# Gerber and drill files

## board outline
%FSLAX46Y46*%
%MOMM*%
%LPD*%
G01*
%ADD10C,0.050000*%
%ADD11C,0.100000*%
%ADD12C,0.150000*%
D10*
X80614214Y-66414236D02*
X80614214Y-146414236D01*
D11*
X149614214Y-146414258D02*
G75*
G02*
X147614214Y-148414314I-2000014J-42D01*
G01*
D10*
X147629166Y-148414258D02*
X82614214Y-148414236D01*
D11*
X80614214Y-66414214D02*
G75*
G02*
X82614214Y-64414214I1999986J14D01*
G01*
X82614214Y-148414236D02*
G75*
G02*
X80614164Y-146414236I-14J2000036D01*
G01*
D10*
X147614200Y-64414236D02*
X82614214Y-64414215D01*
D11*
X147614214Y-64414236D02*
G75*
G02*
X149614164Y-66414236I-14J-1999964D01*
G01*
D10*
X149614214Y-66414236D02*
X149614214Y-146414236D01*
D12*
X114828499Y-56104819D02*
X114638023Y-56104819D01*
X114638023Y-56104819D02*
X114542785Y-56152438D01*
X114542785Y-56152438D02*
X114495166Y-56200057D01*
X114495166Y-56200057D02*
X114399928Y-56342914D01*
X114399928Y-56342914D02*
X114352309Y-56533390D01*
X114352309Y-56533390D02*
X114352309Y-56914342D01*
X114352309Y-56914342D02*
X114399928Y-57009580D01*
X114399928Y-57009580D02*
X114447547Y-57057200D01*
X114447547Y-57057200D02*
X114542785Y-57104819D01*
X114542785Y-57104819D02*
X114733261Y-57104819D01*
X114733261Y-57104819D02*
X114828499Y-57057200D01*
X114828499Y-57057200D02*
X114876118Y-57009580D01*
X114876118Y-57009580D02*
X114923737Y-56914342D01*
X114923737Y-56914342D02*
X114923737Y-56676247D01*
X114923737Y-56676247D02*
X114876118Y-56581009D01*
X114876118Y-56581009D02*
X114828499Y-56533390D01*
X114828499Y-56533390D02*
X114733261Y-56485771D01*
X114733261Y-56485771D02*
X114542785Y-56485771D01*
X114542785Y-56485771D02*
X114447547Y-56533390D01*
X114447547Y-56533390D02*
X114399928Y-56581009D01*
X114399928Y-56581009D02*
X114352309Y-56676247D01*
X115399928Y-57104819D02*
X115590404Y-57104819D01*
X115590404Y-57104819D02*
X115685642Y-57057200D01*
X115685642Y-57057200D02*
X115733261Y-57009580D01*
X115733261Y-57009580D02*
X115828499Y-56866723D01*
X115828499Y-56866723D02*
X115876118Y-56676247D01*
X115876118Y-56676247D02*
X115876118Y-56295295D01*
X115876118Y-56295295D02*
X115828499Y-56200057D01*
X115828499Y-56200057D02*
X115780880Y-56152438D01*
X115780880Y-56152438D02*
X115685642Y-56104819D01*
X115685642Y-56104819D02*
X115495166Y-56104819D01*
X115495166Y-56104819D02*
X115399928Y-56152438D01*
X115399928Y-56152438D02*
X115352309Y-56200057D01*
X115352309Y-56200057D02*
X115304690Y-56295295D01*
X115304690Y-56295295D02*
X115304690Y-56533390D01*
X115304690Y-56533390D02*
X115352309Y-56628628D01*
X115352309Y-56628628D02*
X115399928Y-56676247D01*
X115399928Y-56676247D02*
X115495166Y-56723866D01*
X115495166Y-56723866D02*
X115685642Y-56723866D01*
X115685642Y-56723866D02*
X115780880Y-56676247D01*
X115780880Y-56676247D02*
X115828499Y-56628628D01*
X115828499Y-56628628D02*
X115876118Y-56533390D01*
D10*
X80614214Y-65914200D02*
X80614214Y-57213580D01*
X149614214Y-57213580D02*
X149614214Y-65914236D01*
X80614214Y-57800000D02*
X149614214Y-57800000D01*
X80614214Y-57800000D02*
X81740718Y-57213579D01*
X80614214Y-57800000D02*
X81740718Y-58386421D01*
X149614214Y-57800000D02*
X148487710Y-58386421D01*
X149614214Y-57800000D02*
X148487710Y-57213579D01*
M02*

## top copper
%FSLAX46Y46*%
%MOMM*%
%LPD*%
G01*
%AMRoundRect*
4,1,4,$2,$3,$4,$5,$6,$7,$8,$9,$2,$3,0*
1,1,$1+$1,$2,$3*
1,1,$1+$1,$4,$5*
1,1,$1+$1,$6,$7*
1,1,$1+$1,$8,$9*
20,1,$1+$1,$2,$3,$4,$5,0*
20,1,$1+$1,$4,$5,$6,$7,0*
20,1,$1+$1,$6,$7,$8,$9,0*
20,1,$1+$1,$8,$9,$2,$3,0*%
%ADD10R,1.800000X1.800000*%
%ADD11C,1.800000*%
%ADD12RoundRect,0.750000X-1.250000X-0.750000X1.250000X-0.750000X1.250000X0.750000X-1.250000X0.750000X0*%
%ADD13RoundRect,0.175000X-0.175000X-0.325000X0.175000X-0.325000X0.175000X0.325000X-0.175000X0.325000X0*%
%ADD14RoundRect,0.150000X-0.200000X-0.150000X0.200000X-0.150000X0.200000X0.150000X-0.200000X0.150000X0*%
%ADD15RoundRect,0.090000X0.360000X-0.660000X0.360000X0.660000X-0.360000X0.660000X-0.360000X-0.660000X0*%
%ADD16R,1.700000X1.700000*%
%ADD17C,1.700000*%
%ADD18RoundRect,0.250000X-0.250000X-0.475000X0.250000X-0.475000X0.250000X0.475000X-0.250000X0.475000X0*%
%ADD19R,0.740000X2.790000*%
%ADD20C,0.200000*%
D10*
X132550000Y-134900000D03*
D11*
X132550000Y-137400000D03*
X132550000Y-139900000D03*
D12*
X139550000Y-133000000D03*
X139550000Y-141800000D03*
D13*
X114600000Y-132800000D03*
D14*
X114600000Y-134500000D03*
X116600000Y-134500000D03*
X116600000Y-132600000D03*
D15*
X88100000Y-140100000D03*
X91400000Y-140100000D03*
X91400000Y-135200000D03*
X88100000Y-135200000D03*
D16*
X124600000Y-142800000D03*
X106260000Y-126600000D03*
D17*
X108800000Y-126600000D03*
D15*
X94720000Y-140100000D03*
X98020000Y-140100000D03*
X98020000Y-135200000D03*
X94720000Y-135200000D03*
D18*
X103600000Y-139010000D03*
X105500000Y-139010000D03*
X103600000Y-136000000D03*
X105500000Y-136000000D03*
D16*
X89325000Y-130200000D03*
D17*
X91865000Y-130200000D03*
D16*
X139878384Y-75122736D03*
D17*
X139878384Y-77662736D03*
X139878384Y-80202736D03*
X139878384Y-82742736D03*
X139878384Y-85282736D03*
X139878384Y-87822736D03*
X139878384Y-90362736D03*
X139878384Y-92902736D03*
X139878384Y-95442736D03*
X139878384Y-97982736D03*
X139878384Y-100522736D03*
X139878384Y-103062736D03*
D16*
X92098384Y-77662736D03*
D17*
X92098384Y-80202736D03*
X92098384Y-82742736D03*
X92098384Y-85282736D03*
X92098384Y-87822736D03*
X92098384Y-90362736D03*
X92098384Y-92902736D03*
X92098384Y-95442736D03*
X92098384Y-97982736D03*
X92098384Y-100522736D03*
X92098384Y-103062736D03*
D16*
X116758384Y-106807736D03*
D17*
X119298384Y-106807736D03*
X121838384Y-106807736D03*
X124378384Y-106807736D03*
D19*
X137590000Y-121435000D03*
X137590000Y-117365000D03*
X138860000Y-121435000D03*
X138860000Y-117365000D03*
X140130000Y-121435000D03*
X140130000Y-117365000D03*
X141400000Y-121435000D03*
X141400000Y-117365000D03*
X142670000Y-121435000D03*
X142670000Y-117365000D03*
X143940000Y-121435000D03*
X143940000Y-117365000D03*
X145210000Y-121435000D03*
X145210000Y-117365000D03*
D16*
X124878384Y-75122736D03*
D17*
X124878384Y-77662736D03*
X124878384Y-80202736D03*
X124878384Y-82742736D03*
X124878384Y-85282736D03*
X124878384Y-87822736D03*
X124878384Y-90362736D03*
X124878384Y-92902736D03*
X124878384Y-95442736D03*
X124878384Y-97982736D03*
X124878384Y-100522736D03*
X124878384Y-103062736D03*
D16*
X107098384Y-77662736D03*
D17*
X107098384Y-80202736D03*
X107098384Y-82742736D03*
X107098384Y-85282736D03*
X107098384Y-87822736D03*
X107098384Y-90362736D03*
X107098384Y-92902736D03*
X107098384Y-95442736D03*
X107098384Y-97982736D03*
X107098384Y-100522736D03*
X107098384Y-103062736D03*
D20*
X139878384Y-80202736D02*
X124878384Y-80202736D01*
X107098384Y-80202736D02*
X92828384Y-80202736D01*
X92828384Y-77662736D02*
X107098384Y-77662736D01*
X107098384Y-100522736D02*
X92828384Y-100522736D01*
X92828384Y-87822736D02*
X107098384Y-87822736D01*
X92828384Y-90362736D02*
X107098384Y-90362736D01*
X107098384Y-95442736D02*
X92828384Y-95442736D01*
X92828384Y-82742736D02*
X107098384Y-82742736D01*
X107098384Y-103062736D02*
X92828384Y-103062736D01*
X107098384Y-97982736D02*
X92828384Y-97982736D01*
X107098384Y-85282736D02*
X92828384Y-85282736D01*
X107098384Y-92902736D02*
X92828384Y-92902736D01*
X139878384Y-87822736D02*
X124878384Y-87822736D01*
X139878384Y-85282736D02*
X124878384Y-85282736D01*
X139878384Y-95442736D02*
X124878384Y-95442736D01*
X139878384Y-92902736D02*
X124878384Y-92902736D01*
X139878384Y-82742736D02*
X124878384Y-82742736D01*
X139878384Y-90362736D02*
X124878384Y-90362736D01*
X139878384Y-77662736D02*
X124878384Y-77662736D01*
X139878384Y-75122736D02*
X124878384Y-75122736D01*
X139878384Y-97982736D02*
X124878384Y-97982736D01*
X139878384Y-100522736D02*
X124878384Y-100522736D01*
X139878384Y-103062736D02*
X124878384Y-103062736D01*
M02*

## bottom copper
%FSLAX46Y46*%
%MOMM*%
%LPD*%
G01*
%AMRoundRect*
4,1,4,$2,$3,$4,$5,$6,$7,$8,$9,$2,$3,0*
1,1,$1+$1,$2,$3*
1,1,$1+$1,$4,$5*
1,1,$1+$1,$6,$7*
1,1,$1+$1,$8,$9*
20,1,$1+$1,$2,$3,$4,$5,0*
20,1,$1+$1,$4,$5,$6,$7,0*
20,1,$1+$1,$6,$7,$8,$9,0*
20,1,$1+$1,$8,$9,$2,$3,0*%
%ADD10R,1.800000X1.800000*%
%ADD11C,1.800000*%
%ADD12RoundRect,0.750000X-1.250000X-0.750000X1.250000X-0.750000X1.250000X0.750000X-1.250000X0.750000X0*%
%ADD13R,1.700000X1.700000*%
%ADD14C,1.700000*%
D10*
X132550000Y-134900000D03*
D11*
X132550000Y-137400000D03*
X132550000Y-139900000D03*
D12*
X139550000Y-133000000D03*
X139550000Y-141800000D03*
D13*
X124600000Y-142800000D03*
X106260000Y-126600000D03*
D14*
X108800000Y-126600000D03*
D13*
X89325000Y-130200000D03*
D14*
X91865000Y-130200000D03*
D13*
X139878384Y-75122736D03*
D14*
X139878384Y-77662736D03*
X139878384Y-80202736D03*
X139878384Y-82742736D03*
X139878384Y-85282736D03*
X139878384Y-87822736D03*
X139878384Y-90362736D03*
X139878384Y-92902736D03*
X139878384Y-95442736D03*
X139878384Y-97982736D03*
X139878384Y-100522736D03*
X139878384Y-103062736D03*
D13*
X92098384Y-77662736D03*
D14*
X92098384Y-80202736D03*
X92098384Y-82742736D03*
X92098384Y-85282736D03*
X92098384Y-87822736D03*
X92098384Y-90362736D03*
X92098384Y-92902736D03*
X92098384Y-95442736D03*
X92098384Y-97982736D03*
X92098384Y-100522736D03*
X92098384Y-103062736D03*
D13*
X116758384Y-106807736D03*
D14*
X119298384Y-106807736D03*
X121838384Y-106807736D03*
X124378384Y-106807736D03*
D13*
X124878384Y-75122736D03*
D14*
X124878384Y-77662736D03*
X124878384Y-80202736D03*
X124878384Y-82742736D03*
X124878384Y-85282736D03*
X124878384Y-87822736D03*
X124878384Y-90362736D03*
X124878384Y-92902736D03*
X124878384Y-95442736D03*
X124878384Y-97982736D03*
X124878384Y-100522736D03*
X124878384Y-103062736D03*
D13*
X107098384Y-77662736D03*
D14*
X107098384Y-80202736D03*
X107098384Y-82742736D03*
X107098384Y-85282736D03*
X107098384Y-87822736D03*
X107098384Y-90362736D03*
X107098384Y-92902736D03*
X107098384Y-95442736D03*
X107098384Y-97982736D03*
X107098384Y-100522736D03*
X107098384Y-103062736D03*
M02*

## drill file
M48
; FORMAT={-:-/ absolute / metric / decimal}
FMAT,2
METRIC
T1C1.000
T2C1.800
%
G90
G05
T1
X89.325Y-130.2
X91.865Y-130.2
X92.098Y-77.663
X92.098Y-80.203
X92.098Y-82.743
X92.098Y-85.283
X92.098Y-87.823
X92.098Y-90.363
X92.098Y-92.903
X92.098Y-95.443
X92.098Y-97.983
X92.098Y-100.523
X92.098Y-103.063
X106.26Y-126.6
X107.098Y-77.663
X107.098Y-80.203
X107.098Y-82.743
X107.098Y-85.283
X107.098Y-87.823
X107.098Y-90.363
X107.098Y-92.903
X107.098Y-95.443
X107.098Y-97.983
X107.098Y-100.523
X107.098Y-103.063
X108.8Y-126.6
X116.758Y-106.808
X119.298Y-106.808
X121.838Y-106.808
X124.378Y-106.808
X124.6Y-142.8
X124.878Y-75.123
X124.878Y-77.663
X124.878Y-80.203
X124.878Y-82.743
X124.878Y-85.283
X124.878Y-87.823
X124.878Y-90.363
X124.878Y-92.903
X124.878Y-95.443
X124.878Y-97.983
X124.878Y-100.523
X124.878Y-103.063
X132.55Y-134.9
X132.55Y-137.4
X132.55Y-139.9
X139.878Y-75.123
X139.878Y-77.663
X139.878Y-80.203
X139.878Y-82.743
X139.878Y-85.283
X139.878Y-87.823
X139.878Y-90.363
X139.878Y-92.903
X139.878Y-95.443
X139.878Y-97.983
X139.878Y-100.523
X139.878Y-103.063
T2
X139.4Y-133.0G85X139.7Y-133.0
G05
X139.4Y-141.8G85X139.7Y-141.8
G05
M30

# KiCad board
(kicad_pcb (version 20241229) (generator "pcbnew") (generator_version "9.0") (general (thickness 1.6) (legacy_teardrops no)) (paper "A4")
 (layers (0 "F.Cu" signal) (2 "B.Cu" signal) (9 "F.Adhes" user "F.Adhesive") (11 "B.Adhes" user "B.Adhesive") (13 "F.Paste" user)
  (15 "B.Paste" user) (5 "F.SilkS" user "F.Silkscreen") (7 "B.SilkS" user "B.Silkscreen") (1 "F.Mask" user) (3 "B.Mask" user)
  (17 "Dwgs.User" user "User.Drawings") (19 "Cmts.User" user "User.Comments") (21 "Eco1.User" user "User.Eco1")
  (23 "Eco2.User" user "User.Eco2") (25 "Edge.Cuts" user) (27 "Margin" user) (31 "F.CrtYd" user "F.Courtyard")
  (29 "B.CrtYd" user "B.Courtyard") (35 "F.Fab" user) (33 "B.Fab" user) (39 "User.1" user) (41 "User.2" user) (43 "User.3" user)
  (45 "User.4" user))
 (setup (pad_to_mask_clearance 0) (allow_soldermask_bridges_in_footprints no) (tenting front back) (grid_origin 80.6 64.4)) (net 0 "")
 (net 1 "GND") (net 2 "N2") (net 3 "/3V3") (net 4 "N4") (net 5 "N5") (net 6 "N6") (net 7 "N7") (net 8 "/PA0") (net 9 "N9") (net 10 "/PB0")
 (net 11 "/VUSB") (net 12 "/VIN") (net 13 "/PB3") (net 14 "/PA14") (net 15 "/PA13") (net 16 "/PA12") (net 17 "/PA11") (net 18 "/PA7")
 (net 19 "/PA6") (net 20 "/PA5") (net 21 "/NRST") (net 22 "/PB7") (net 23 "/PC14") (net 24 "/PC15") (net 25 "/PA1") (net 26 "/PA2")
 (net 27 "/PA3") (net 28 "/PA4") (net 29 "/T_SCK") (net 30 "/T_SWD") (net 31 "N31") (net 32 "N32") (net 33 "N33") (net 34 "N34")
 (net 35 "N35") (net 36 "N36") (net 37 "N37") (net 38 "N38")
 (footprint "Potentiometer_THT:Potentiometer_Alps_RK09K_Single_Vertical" (layer "F.Cu") (at 132.55 134.9)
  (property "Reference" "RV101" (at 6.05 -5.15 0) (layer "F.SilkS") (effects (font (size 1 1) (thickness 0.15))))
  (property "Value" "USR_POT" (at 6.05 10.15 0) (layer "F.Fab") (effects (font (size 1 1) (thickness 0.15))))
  (pad "1" thru_hole rect (at 0 0) (size 1.8 1.8) (drill 1) (layers "*.Cu" "*.Mask") (remove_unused_layers no) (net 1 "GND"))
  (pad "2" thru_hole circle (at 0 2.5) (size 1.8 1.8) (drill 1) (layers "*.Cu" "*.Mask") (remove_unused_layers no) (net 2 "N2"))
  (pad "3" thru_hole circle (at 0 5) (size 1.8 1.8) (drill 1) (layers "*.Cu" "*.Mask") (remove_unused_layers no) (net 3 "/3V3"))
  (pad "MP" thru_hole roundrect (at 7 -1.9) (size 4 3) (drill oval 2.1 1.8) (layers "*.Cu" "*.Mask") (remove_unused_layers no)
   (roundrect_rratio 0.25))
  (pad "MP" thru_hole roundrect (at 7 6.9) (size 4 3) (drill oval 2.1 1.8) (layers "*.Cu" "*.Mask") (remove_unused_layers no)
   (roundrect_rratio 0.25)))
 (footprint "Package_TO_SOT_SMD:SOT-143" (layer "F.Cu") (at 115.6 133.55)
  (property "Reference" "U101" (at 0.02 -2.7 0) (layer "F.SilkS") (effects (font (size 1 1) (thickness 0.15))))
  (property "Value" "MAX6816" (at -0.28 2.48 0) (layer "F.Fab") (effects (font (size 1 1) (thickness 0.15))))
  (pad "1" smd roundrect (at -1 -0.75) (size 0.7 1) (layers "F.Cu" "F.Mask" "F.Paste") (roundrect_rratio 0.25) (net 1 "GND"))
  (pad "2" smd roundrect (at -1 0.95) (size 0.7 0.6) (layers "F.Cu" "F.Mask" "F.Paste") (roundrect_rratio 0.25) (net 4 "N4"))
  (pad "3" smd roundrect (at 1 0.95) (size 0.7 0.6) (layers "F.Cu" "F.Mask" "F.Paste") (roundrect_rratio 0.25) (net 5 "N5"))
  (pad "4" smd roundrect (at 1 -0.95) (size 0.7 0.6) (layers "F.Cu" "F.Mask" "F.Paste") (roundrect_rratio 0.25) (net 3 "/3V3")))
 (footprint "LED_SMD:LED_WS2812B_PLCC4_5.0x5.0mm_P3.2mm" (layer "F.Cu") (at 89.75 137.65 90)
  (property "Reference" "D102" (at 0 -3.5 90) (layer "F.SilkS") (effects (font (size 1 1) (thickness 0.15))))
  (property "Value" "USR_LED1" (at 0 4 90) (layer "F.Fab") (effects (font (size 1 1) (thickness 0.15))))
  (pad "1" smd roundrect (at -2.45 -1.65 90) (size 1.5 0.9) (layers "F.Cu" "F.Mask" "F.Paste") (roundrect_rratio 0.1) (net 3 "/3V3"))
  (pad "2" smd roundrect (at -2.45 1.65 90) (size 1.5 0.9) (layers "F.Cu" "F.Mask" "F.Paste") (roundrect_rratio 0.1) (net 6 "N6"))
  (pad "3" smd roundrect (at 2.45 1.65 90) (size 1.5 0.9) (layers "F.Cu" "F.Mask" "F.Paste") (roundrect_rratio 0.1) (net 1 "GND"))
  (pad "4" smd roundrect (at 2.45 -1.65 90) (size 1.5 0.9) (layers "F.Cu" "F.Mask" "F.Paste") (roundrect_rratio 0.1) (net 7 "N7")))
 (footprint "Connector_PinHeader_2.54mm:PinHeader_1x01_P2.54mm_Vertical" (layer "F.Cu") (at 124.6 142.8)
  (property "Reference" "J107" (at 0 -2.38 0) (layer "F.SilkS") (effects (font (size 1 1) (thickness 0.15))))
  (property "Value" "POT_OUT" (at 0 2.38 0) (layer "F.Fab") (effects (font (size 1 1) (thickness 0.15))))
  (pad "1" thru_hole rect (at 0 0) (size 1.7 1.7) (drill 1) (layers "*.Cu" "*.Mask") (remove_unused_layers no) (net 2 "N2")))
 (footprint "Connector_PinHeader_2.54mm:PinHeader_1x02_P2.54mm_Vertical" (layer "F.Cu") (at 106.26 126.6 90)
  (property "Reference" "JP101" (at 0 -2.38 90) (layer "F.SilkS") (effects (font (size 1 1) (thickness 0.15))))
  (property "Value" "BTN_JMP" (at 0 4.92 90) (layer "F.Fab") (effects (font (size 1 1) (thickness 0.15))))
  (pad "1" thru_hole rect (at 0 0 90) (size 1.7 1.7) (drill 1) (layers "*.Cu" "*.Mask") (remove_unused_layers no) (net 5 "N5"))
  (pad "2" thru_hole circle (at 0 2.54 90) (size 1.7 1.7) (drill 1) (layers "*.Cu" "*.Mask") (remove_unused_layers no) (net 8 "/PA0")))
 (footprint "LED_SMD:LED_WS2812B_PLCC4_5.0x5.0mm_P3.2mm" (layer "F.Cu") (at 96.37 137.65 90)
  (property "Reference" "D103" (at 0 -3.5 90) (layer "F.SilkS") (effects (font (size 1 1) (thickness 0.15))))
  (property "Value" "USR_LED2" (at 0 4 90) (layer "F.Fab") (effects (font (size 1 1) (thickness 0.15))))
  (pad "1" smd roundrect (at -2.45 -1.65 90) (size 1.5 0.9) (layers "F.Cu" "F.Mask" "F.Paste") (roundrect_rratio 0.1) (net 3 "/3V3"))
  (pad "2" smd roundrect (at -2.45 1.65 90) (size 1.5 0.9) (layers "F.Cu" "F.Mask" "F.Paste") (roundrect_rratio 0.1) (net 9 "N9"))
  (pad "3" smd roundrect (at 2.45 1.65 90) (size 1.5 0.9) (layers "F.Cu" "F.Mask" "F.Paste") (roundrect_rratio 0.1) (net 1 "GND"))
  (pad "4" smd roundrect (at 2.45 -1.65 90) (size 1.5 0.9) (layers "F.Cu" "F.Mask" "F.Paste") (roundrect_rratio 0.1) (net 6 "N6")))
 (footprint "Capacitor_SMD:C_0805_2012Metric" (layer "F.Cu") (at 104.55 139.01)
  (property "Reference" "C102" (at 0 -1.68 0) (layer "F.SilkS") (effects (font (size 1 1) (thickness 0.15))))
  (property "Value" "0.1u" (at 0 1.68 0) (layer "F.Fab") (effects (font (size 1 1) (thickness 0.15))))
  (pad "1" smd roundrect (at -0.95 0) (size 1 1.45) (layers "F.Cu" "F.Mask" "F.Paste") (roundrect_rratio 0.25) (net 3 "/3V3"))
  (pad "2" smd roundrect (at 0.95 0) (size 1 1.45) (layers "F.Cu" "F.Mask" "F.Paste") (roundrect_rratio 0.25) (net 1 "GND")))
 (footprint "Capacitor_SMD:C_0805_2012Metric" (layer "F.Cu") (at 104.55 136)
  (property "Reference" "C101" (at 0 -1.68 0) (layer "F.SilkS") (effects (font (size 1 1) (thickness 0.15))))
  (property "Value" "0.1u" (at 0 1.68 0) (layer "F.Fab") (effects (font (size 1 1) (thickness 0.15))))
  (pad "1" smd roundrect (at -0.95 0) (size 1 1.45) (layers "F.Cu" "F.Mask" "F.Paste") (roundrect_rratio 0.25) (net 3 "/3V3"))
  (pad "2" smd roundrect (at 0.95 0) (size 1 1.45) (layers "F.Cu" "F.Mask" "F.Paste") (roundrect_rratio 0.25) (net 1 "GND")))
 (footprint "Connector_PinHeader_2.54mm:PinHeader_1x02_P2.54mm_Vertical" (layer "F.Cu") (at 89.325 130.2 90)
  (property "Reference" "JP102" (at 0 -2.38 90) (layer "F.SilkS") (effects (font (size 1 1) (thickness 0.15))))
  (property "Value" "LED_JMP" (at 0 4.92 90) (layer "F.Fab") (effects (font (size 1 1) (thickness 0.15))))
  (pad "1" thru_hole rect (at 0 0 90) (size 1.7 1.7) (drill 1) (layers "*.Cu" "*.Mask") (remove_unused_layers no) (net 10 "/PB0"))
  (pad "2" thru_hole circle (at 0 2.54 90) (size 1.7 1.7) (drill 1) (layers "*.Cu" "*.Mask") (remove_unused_layers no) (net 7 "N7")))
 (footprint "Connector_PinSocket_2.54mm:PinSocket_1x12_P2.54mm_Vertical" (layer "F.Cu") (at 139.878384 75.122736)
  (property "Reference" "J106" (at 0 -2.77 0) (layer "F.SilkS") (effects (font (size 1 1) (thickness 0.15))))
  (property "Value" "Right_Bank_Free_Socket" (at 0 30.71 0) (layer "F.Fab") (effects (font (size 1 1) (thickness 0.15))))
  (pad "1" thru_hole rect (at 0 0) (size 1.7 1.7) (drill 1) (layers "*.Cu" "*.Mask") (remove_unused_layers no) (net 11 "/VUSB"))
  (pad "2" thru_hole circle (at 0 2.54) (size 1.7 1.7) (drill 1) (layers "*.Cu" "*.Mask") (remove_unused_layers no) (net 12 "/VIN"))
  (pad "3" thru_hole circle (at 0 5.08) (size 1.7 1.7) (drill 1) (layers "*.Cu" "*.Mask") (remove_unused_layers no) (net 1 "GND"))
  (pad "4" thru_hole circle (at 0 7.62) (size 1.7 1.7) (drill 1) (layers "*.Cu" "*.Mask") (remove_unused_layers no) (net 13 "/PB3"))
  (pad "5" thru_hole circle (at 0 10.16) (size 1.7 1.7) (drill 1) (layers "*.Cu" "*.Mask") (remove_unused_layers no) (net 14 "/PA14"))
  (pad "6" thru_hole circle (at 0 12.7) (size 1.7 1.7) (drill 1) (layers "*.Cu" "*.Mask") (remove_unused_layers no) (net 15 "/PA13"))
  (pad "7" thru_hole circle (at 0 15.24) (size 1.7 1.7) (drill 1) (layers "*.Cu" "*.Mask") (remove_unused_layers no) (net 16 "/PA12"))
  (pad "8" thru_hole circle (at 0 17.78) (size 1.7 1.7) (drill 1) (layers "*.Cu" "*.Mask") (remove_unused_layers no) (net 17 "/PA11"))
  (pad "9" thru_hole circle (at 0 20.32) (size 1.7 1.7) (drill 1) (layers "*.Cu" "*.Mask") (remove_unused_layers no) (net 10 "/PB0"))
  (pad "10" thru_hole circle (at 0 22.86) (size 1.7 1.7) (drill 1) (layers "*.Cu" "*.Mask") (remove_unused_layers no) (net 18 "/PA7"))
  (pad "11" thru_hole circle (at 0 25.4) (size 1.7 1.7) (drill 1) (layers "*.Cu" "*.Mask") (remove_unused_layers no) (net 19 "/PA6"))
  (pad "12" thru_hole circle (at 0 27.94) (size 1.7 1.7) (drill 1) (layers "*.Cu" "*.Mask") (remove_unused_layers no) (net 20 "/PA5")))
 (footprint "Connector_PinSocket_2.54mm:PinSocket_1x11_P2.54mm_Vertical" (layer "F.Cu") (at 92.098384 77.662736)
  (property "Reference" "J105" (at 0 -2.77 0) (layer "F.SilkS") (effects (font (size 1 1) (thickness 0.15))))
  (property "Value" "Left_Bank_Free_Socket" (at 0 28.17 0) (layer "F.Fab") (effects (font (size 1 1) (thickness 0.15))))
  (pad "1" thru_hole rect (at 0 0) (size 1.7 1.7) (drill 1) (layers "*.Cu" "*.Mask") (remove_unused_layers no) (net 3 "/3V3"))
  (pad "2" thru_hole circle (at 0 2.54) (size 1.7 1.7) (drill 1) (layers "*.Cu" "*.Mask") (remove_unused_layers no) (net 1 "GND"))
  (pad "3" thru_hole circle (at 0 5.08) (size 1.7 1.7) (drill 1) (layers "*.Cu" "*.Mask") (remove_unused_layers no) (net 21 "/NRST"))
  (pad "4" thru_hole circle (at 0 7.62) (size 1.7 1.7) (drill 1) (layers "*.Cu" "*.Mask") (remove_unused_layers no) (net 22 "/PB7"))
  (pad "5" thru_hole circle (at 0 10.16) (size 1.7 1.7) (drill 1) (layers "*.Cu" "*.Mask") (remove_unused_layers no) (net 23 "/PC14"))
  (pad "6" thru_hole circle (at 0 12.7) (size 1.7 1.7) (drill 1) (layers "*.Cu" "*.Mask") (remove_unused_layers no) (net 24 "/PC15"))
  (pad "7" thru_hole circle (at 0 15.24) (size 1.7 1.7) (drill 1) (layers "*.Cu" "*.Mask") (remove_unused_layers no) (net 8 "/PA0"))
  (pad "8" thru_hole circle (at 0 17.78) (size 1.7 1.7) (drill 1) (layers "*.Cu" "*.Mask") (remove_unused_layers no) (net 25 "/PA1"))
  (pad "9" thru_hole circle (at 0 20.32) (size 1.7 1.7) (drill 1) (layers "*.Cu" "*.Mask") (remove_unused_layers no) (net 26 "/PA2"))
  (pad "10" thru_hole circle (at 0 22.86) (size 1.7 1.7) (drill 1) (layers "*.Cu" "*.Mask") (remove_unused_layers no) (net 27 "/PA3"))
  (pad "11" thru_hole circle (at 0 25.4) (size 1.7 1.7) (drill 1) (layers "*.Cu" "*.Mask") (remove_unused_layers no) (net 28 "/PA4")))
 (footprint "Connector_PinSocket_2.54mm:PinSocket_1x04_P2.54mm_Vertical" (layer "F.Cu") (at 116.758384 106.807736 90)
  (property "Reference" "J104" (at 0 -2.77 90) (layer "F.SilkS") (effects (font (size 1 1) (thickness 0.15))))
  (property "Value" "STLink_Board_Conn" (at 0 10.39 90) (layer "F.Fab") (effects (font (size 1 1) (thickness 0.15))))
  (pad "1" thru_hole rect (at 0 0 90) (size 1.7 1.7) (drill 1) (layers "*.Cu" "*.Mask") (remove_unused_layers no) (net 3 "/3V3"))
  (pad "2" thru_hole circle (at 0 2.54 90) (size 1.7 1.7) (drill 1) (layers "*.Cu" "*.Mask") (remove_unused_layers no) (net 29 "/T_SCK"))
  (pad "3" thru_hole circle (at 0 5.08 90) (size 1.7 1.7) (drill 1) (layers "*.Cu" "*.Mask") (remove_unused_layers no) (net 1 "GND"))
  (pad "4" thru_hole circle (at 0 7.62 90) (size 1.7 1.7) (drill 1) (layers "*.Cu" "*.Mask") (remove_unused_layers no) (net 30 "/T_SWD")))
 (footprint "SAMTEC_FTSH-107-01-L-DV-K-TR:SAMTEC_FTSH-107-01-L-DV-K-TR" (layer "F.Cu") (at 141.4 119.4)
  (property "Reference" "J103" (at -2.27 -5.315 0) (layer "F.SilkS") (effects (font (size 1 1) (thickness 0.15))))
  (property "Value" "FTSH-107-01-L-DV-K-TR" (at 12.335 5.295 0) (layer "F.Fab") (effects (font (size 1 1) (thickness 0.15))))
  (pad "1" smd rect (at -3.81 2.035) (size 0.74 2.79) (layers "F.Cu" "F.Mask" "F.Paste") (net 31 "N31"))
  (pad "2" smd rect (at -3.81 -2.035) (size 0.74 2.79) (layers "F.Cu" "F.Mask" "F.Paste") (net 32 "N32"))
  (pad "3" smd rect (at -2.54 2.035) (size 0.74 2.79) (layers "F.Cu" "F.Mask" "F.Paste") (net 3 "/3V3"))
  (pad "4" smd rect (at -2.54 -2.035) (size 0.74 2.79) (layers "F.Cu" "F.Mask" "F.Paste") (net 30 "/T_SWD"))
  (pad "5" smd rect (at -1.27 2.035) (size 0.74 2.79) (layers "F.Cu" "F.Mask" "F.Paste") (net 1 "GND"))
  (pad "6" smd rect (at -1.27 -2.035) (size 0.74 2.79) (layers "F.Cu" "F.Mask" "F.Paste") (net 29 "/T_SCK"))
  (pad "7" smd rect (at 0 2.035) (size 0.74 2.79) (layers "F.Cu" "F.Mask" "F.Paste") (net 1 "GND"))
  (pad "8" smd rect (at 0 -2.035) (size 0.74 2.79) (layers "F.Cu" "F.Mask" "F.Paste") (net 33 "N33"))
  (pad "9" smd rect (at 1.27 2.035) (size 0.74 2.79) (layers "F.Cu" "F.Mask" "F.Paste") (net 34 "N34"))
  (pad "10" smd rect (at 1.27 -2.035) (size 0.74 2.79) (layers "F.Cu" "F.Mask" "F.Paste") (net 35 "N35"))
  (pad "11" smd rect (at 2.54 2.035) (size 0.74 2.79) (layers "F.Cu" "F.Mask" "F.Paste") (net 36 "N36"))
  (pad "12" smd rect (at 2.54 -2.035) (size 0.74 2.79) (layers "F.Cu" "F.Mask" "F.Paste") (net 21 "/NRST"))
  (pad "13" smd rect (at 3.81 2.035) (size 0.74 2.79) (layers "F.Cu" "F.Mask" "F.Paste") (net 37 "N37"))
  (pad "14" smd rect (at 3.81 -2.035) (size 0.74 2.79) (layers "F.Cu" "F.Mask" "F.Paste") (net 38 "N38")))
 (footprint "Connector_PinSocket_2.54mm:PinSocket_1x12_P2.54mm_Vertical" (layer "F.Cu") (at 124.878384 75.122736)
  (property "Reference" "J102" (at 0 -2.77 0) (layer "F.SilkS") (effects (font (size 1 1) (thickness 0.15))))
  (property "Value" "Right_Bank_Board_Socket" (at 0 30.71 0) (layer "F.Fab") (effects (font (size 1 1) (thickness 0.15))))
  (pad "1" thru_hole rect (at 0 0) (size 1.7 1.7) (drill 1) (layers "*.Cu" "*.Mask") (remove_unused_layers no) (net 11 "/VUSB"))
  (pad "2" thru_hole circle (at 0 2.54) (size 1.7 1.7) (drill 1) (layers "*.Cu" "*.Mask") (remove_unused_layers no) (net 12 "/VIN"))
  (pad "3" thru_hole circle (at 0 5.08) (size 1.7 1.7) (drill 1) (layers "*.Cu" "*.Mask") (remove_unused_layers no) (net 1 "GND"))
  (pad "4" thru_hole circle (at 0 7.62) (size 1.7 1.7) (drill 1) (layers "*.Cu" "*.Mask") (remove_unused_layers no) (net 13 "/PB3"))
  (pad "5" thru_hole circle (at 0 10.16) (size 1.7 1.7) (drill 1) (layers "*.Cu" "*.Mask") (remove_unused_layers no) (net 14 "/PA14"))
  (pad "6" thru_hole circle (at 0 12.7) (size 1.7 1.7) (drill 1) (layers "*.Cu" "*.Mask") (remove_unused_layers no) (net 15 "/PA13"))
  (pad "7" thru_hole circle (at 0 15.24) (size 1.7 1.7) (drill 1) (layers "*.Cu" "*.Mask") (remove_unused_layers no) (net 16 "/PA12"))
  (pad "8" thru_hole circle (at 0 17.78) (size 1.7 1.7) (drill 1) (layers "*.Cu" "*.Mask") (remove_unused_layers no) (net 17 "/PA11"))
  (pad "9" thru_hole circle (at 0 20.32) (size 1.7 1.7) (drill 1) (layers "*.Cu" "*.Mask") (remove_unused_layers no) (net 10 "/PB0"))
  (pad "10" thru_hole circle (at 0 22.86) (size 1.7 1.7) (drill 1) (layers "*.Cu" "*.Mask") (remove_unused_layers no) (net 18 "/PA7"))
  (pad "11" thru_hole circle (at 0 25.4) (size 1.7 1.7) (drill 1) (layers "*.Cu" "*.Mask") (remove_unused_layers no) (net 19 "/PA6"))
  (pad "12" thru_hole circle (at 0 27.94) (size 1.7 1.7) (drill 1) (layers "*.Cu" "*.Mask") (remove_unused_layers no) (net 20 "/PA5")))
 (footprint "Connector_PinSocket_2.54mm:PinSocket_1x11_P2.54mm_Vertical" (layer "F.Cu") (at 107.098384 77.662736)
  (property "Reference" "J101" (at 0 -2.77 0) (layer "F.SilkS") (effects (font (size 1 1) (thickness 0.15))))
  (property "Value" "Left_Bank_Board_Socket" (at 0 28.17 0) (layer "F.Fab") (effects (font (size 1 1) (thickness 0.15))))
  (pad "1" thru_hole rect (at 0 0) (size 1.7 1.7) (drill 1) (layers "*.Cu" "*.Mask") (remove_unused_layers no) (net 3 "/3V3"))
  (pad "2" thru_hole circle (at 0 2.54) (size 1.7 1.7) (drill 1) (layers "*.Cu" "*.Mask") (remove_unused_layers no) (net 1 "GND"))
  (pad "3" thru_hole circle (at 0 5.08) (size 1.7 1.7) (drill 1) (layers "*.Cu" "*.Mask") (remove_unused_layers no) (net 21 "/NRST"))
  (pad "4" thru_hole circle (at 0 7.62) (size 1.7 1.7) (drill 1) (layers "*.Cu" "*.Mask") (remove_unused_layers no) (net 22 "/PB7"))
  (pad "5" thru_hole circle (at 0 10.16) (size 1.7 1.7) (drill 1) (layers "*.Cu" "*.Mask") (remove_unused_layers no) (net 23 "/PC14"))
  (pad "6" thru_hole circle (at 0 12.7) (size 1.7 1.7) (drill 1) (layers "*.Cu" "*.Mask") (remove_unused_layers no) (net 24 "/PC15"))
  (pad "7" thru_hole circle (at 0 15.24) (size 1.7 1.7) (drill 1) (layers "*.Cu" "*.Mask") (remove_unused_layers no) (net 8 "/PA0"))
  (pad "8" thru_hole circle (at 0 17.78) (size 1.7 1.7) (drill 1) (layers "*.Cu" "*.Mask") (remove_unused_layers no) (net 25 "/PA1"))
  (pad "9" thru_hole circle (at 0 20.32) (size 1.7 1.7) (drill 1) (layers "*.Cu" "*.Mask") (remove_unused_layers no) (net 26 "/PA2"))
  (pad "10" thru_hole circle (at 0 22.86) (size 1.7 1.7) (drill 1) (layers "*.Cu" "*.Mask") (remove_unused_layers no) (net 27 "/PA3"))
  (pad "11" thru_hole circle (at 0 25.4) (size 1.7 1.7) (drill 1) (layers "*.Cu" "*.Mask") (remove_unused_layers no) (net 28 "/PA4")))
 (gr_line (start 80.614214 66.414236) (end 80.614214 146.414236) (stroke (width 0.05) (type solid)) (layer "Edge.Cuts"))
 (gr_arc (start 149.614214 146.414258) (mid 149.028428 147.828472) (end 147.614214 148.414258) (stroke (width 0.1) (type solid))
  (layer "Edge.Cuts"))
 (gr_line (start 147.629166 148.414258) (end 82.614214 148.414236) (stroke (width 0.05) (type default)) (layer "Edge.Cuts"))
 (gr_arc (start 80.614214 66.414214) (mid 81.2 65) (end 82.614214 64.414214) (stroke (width 0.1) (type solid)) (layer "Edge.Cuts"))
 (gr_arc (start 82.614214 148.414236) (mid 81.2 147.82845) (end 80.614214 146.414236) (stroke (width 0.1) (type solid)) (layer "Edge.Cuts"))
 (gr_line (start 147.6142 64.414236) (end 82.614214 64.414215) (stroke (width 0.05) (type default)) (layer "Edge.Cuts"))
 (gr_arc (start 147.614214 64.414236) (mid 149.028428 65.000022) (end 149.614214 66.414236) (stroke (width 0.1) (type solid))
  (layer "Edge.Cuts"))
 (gr_line (start 149.614214 66.414236) (end 149.614214 146.414236) (stroke (width 0.05) (type solid)) (layer "Edge.Cuts"))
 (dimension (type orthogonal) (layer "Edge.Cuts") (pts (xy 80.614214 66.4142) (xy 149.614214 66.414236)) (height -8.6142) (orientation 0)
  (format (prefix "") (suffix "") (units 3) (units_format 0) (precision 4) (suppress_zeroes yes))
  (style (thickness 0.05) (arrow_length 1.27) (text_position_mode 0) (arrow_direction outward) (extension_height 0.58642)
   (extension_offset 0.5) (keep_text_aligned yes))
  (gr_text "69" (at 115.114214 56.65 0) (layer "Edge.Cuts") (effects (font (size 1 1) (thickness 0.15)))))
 (segment (start 139.878384 80.202736) (end 124.878384 80.202736) (width 0.2) (layer "F.Cu") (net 1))
 (segment (start 107.098384 80.202736) (end 92.828384 80.202736) (width 0.2) (layer "F.Cu") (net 1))
 (segment (start 92.828384 77.662736) (end 107.098384 77.662736) (width 0.2) (layer "F.Cu") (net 3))
 (segment (start 107.098384 100.522736) (end 92.828384 100.522736) (width 0.2) (layer "F.Cu") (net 27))
 (segment (start 92.828384 87.822736) (end 107.098384 87.822736) (width 0.2) (layer "F.Cu") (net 23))
 (segment (start 92.828384 90.362736) (end 107.098384 90.362736) (width 0.2) (layer "F.Cu") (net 24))
 (segment (start 107.098384 95.442736) (end 92.828384 95.442736) (width 0.2) (layer "F.Cu") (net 25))
 (segment (start 92.828384 82.742736) (end 107.098384 82.742736) (width 0.2) (layer "F.Cu") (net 21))
 (segment (start 107.098384 103.062736) (end 92.828384 103.062736) (width 0.2) (layer "F.Cu") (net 28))
 (segment (start 107.098384 97.982736) (end 92.828384 97.982736) (width 0.2) (layer "F.Cu") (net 26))
 (segment (start 107.098384 85.282736) (end 92.828384 85.282736) (width 0.2) (layer "F.Cu") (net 22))
 (segment (start 107.098384 92.902736) (end 92.828384 92.902736) (width 0.2) (layer "F.Cu") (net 8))
 (segment (start 139.878384 87.822736) (end 124.878384 87.822736) (width 0.2) (layer "F.Cu") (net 15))
 (segment (start 139.878384 85.282736) (end 124.878384 85.282736) (width 0.2) (layer "F.Cu") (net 14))
 (segment (start 139.878384 95.442736) (end 124.878384 95.442736) (width 0.2) (layer "F.Cu") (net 10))
 (segment (start 139.878384 92.902736) (end 124.878384 92.902736) (width 0.2) (layer "F.Cu") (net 17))
 (segment (start 139.878384 82.742736) (end 124.878384 82.742736) (width 0.2) (layer "F.Cu") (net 13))
 (segment (start 139.878384 90.362736) (end 124.878384 90.362736) (width 0.2) (layer "F.Cu") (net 16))
 (segment (start 139.878384 77.662736) (end 124.878384 77.662736) (width 0.2) (layer "F.Cu") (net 12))
 (segment (start 139.878384 75.122736) (end 124.878384 75.122736) (width 0.2) (layer "F.Cu") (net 11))
 (segment (start 139.878384 97.982736) (end 124.878384 97.982736) (width 0.2) (layer "F.Cu") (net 18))
 (segment (start 139.878384 100.522736) (end 124.878384 100.522736) (width 0.2) (layer "F.Cu") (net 19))
 (segment (start 139.878384 103.062736) (end 124.878384 103.062736) (width 0.2) (layer "F.Cu") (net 20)))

